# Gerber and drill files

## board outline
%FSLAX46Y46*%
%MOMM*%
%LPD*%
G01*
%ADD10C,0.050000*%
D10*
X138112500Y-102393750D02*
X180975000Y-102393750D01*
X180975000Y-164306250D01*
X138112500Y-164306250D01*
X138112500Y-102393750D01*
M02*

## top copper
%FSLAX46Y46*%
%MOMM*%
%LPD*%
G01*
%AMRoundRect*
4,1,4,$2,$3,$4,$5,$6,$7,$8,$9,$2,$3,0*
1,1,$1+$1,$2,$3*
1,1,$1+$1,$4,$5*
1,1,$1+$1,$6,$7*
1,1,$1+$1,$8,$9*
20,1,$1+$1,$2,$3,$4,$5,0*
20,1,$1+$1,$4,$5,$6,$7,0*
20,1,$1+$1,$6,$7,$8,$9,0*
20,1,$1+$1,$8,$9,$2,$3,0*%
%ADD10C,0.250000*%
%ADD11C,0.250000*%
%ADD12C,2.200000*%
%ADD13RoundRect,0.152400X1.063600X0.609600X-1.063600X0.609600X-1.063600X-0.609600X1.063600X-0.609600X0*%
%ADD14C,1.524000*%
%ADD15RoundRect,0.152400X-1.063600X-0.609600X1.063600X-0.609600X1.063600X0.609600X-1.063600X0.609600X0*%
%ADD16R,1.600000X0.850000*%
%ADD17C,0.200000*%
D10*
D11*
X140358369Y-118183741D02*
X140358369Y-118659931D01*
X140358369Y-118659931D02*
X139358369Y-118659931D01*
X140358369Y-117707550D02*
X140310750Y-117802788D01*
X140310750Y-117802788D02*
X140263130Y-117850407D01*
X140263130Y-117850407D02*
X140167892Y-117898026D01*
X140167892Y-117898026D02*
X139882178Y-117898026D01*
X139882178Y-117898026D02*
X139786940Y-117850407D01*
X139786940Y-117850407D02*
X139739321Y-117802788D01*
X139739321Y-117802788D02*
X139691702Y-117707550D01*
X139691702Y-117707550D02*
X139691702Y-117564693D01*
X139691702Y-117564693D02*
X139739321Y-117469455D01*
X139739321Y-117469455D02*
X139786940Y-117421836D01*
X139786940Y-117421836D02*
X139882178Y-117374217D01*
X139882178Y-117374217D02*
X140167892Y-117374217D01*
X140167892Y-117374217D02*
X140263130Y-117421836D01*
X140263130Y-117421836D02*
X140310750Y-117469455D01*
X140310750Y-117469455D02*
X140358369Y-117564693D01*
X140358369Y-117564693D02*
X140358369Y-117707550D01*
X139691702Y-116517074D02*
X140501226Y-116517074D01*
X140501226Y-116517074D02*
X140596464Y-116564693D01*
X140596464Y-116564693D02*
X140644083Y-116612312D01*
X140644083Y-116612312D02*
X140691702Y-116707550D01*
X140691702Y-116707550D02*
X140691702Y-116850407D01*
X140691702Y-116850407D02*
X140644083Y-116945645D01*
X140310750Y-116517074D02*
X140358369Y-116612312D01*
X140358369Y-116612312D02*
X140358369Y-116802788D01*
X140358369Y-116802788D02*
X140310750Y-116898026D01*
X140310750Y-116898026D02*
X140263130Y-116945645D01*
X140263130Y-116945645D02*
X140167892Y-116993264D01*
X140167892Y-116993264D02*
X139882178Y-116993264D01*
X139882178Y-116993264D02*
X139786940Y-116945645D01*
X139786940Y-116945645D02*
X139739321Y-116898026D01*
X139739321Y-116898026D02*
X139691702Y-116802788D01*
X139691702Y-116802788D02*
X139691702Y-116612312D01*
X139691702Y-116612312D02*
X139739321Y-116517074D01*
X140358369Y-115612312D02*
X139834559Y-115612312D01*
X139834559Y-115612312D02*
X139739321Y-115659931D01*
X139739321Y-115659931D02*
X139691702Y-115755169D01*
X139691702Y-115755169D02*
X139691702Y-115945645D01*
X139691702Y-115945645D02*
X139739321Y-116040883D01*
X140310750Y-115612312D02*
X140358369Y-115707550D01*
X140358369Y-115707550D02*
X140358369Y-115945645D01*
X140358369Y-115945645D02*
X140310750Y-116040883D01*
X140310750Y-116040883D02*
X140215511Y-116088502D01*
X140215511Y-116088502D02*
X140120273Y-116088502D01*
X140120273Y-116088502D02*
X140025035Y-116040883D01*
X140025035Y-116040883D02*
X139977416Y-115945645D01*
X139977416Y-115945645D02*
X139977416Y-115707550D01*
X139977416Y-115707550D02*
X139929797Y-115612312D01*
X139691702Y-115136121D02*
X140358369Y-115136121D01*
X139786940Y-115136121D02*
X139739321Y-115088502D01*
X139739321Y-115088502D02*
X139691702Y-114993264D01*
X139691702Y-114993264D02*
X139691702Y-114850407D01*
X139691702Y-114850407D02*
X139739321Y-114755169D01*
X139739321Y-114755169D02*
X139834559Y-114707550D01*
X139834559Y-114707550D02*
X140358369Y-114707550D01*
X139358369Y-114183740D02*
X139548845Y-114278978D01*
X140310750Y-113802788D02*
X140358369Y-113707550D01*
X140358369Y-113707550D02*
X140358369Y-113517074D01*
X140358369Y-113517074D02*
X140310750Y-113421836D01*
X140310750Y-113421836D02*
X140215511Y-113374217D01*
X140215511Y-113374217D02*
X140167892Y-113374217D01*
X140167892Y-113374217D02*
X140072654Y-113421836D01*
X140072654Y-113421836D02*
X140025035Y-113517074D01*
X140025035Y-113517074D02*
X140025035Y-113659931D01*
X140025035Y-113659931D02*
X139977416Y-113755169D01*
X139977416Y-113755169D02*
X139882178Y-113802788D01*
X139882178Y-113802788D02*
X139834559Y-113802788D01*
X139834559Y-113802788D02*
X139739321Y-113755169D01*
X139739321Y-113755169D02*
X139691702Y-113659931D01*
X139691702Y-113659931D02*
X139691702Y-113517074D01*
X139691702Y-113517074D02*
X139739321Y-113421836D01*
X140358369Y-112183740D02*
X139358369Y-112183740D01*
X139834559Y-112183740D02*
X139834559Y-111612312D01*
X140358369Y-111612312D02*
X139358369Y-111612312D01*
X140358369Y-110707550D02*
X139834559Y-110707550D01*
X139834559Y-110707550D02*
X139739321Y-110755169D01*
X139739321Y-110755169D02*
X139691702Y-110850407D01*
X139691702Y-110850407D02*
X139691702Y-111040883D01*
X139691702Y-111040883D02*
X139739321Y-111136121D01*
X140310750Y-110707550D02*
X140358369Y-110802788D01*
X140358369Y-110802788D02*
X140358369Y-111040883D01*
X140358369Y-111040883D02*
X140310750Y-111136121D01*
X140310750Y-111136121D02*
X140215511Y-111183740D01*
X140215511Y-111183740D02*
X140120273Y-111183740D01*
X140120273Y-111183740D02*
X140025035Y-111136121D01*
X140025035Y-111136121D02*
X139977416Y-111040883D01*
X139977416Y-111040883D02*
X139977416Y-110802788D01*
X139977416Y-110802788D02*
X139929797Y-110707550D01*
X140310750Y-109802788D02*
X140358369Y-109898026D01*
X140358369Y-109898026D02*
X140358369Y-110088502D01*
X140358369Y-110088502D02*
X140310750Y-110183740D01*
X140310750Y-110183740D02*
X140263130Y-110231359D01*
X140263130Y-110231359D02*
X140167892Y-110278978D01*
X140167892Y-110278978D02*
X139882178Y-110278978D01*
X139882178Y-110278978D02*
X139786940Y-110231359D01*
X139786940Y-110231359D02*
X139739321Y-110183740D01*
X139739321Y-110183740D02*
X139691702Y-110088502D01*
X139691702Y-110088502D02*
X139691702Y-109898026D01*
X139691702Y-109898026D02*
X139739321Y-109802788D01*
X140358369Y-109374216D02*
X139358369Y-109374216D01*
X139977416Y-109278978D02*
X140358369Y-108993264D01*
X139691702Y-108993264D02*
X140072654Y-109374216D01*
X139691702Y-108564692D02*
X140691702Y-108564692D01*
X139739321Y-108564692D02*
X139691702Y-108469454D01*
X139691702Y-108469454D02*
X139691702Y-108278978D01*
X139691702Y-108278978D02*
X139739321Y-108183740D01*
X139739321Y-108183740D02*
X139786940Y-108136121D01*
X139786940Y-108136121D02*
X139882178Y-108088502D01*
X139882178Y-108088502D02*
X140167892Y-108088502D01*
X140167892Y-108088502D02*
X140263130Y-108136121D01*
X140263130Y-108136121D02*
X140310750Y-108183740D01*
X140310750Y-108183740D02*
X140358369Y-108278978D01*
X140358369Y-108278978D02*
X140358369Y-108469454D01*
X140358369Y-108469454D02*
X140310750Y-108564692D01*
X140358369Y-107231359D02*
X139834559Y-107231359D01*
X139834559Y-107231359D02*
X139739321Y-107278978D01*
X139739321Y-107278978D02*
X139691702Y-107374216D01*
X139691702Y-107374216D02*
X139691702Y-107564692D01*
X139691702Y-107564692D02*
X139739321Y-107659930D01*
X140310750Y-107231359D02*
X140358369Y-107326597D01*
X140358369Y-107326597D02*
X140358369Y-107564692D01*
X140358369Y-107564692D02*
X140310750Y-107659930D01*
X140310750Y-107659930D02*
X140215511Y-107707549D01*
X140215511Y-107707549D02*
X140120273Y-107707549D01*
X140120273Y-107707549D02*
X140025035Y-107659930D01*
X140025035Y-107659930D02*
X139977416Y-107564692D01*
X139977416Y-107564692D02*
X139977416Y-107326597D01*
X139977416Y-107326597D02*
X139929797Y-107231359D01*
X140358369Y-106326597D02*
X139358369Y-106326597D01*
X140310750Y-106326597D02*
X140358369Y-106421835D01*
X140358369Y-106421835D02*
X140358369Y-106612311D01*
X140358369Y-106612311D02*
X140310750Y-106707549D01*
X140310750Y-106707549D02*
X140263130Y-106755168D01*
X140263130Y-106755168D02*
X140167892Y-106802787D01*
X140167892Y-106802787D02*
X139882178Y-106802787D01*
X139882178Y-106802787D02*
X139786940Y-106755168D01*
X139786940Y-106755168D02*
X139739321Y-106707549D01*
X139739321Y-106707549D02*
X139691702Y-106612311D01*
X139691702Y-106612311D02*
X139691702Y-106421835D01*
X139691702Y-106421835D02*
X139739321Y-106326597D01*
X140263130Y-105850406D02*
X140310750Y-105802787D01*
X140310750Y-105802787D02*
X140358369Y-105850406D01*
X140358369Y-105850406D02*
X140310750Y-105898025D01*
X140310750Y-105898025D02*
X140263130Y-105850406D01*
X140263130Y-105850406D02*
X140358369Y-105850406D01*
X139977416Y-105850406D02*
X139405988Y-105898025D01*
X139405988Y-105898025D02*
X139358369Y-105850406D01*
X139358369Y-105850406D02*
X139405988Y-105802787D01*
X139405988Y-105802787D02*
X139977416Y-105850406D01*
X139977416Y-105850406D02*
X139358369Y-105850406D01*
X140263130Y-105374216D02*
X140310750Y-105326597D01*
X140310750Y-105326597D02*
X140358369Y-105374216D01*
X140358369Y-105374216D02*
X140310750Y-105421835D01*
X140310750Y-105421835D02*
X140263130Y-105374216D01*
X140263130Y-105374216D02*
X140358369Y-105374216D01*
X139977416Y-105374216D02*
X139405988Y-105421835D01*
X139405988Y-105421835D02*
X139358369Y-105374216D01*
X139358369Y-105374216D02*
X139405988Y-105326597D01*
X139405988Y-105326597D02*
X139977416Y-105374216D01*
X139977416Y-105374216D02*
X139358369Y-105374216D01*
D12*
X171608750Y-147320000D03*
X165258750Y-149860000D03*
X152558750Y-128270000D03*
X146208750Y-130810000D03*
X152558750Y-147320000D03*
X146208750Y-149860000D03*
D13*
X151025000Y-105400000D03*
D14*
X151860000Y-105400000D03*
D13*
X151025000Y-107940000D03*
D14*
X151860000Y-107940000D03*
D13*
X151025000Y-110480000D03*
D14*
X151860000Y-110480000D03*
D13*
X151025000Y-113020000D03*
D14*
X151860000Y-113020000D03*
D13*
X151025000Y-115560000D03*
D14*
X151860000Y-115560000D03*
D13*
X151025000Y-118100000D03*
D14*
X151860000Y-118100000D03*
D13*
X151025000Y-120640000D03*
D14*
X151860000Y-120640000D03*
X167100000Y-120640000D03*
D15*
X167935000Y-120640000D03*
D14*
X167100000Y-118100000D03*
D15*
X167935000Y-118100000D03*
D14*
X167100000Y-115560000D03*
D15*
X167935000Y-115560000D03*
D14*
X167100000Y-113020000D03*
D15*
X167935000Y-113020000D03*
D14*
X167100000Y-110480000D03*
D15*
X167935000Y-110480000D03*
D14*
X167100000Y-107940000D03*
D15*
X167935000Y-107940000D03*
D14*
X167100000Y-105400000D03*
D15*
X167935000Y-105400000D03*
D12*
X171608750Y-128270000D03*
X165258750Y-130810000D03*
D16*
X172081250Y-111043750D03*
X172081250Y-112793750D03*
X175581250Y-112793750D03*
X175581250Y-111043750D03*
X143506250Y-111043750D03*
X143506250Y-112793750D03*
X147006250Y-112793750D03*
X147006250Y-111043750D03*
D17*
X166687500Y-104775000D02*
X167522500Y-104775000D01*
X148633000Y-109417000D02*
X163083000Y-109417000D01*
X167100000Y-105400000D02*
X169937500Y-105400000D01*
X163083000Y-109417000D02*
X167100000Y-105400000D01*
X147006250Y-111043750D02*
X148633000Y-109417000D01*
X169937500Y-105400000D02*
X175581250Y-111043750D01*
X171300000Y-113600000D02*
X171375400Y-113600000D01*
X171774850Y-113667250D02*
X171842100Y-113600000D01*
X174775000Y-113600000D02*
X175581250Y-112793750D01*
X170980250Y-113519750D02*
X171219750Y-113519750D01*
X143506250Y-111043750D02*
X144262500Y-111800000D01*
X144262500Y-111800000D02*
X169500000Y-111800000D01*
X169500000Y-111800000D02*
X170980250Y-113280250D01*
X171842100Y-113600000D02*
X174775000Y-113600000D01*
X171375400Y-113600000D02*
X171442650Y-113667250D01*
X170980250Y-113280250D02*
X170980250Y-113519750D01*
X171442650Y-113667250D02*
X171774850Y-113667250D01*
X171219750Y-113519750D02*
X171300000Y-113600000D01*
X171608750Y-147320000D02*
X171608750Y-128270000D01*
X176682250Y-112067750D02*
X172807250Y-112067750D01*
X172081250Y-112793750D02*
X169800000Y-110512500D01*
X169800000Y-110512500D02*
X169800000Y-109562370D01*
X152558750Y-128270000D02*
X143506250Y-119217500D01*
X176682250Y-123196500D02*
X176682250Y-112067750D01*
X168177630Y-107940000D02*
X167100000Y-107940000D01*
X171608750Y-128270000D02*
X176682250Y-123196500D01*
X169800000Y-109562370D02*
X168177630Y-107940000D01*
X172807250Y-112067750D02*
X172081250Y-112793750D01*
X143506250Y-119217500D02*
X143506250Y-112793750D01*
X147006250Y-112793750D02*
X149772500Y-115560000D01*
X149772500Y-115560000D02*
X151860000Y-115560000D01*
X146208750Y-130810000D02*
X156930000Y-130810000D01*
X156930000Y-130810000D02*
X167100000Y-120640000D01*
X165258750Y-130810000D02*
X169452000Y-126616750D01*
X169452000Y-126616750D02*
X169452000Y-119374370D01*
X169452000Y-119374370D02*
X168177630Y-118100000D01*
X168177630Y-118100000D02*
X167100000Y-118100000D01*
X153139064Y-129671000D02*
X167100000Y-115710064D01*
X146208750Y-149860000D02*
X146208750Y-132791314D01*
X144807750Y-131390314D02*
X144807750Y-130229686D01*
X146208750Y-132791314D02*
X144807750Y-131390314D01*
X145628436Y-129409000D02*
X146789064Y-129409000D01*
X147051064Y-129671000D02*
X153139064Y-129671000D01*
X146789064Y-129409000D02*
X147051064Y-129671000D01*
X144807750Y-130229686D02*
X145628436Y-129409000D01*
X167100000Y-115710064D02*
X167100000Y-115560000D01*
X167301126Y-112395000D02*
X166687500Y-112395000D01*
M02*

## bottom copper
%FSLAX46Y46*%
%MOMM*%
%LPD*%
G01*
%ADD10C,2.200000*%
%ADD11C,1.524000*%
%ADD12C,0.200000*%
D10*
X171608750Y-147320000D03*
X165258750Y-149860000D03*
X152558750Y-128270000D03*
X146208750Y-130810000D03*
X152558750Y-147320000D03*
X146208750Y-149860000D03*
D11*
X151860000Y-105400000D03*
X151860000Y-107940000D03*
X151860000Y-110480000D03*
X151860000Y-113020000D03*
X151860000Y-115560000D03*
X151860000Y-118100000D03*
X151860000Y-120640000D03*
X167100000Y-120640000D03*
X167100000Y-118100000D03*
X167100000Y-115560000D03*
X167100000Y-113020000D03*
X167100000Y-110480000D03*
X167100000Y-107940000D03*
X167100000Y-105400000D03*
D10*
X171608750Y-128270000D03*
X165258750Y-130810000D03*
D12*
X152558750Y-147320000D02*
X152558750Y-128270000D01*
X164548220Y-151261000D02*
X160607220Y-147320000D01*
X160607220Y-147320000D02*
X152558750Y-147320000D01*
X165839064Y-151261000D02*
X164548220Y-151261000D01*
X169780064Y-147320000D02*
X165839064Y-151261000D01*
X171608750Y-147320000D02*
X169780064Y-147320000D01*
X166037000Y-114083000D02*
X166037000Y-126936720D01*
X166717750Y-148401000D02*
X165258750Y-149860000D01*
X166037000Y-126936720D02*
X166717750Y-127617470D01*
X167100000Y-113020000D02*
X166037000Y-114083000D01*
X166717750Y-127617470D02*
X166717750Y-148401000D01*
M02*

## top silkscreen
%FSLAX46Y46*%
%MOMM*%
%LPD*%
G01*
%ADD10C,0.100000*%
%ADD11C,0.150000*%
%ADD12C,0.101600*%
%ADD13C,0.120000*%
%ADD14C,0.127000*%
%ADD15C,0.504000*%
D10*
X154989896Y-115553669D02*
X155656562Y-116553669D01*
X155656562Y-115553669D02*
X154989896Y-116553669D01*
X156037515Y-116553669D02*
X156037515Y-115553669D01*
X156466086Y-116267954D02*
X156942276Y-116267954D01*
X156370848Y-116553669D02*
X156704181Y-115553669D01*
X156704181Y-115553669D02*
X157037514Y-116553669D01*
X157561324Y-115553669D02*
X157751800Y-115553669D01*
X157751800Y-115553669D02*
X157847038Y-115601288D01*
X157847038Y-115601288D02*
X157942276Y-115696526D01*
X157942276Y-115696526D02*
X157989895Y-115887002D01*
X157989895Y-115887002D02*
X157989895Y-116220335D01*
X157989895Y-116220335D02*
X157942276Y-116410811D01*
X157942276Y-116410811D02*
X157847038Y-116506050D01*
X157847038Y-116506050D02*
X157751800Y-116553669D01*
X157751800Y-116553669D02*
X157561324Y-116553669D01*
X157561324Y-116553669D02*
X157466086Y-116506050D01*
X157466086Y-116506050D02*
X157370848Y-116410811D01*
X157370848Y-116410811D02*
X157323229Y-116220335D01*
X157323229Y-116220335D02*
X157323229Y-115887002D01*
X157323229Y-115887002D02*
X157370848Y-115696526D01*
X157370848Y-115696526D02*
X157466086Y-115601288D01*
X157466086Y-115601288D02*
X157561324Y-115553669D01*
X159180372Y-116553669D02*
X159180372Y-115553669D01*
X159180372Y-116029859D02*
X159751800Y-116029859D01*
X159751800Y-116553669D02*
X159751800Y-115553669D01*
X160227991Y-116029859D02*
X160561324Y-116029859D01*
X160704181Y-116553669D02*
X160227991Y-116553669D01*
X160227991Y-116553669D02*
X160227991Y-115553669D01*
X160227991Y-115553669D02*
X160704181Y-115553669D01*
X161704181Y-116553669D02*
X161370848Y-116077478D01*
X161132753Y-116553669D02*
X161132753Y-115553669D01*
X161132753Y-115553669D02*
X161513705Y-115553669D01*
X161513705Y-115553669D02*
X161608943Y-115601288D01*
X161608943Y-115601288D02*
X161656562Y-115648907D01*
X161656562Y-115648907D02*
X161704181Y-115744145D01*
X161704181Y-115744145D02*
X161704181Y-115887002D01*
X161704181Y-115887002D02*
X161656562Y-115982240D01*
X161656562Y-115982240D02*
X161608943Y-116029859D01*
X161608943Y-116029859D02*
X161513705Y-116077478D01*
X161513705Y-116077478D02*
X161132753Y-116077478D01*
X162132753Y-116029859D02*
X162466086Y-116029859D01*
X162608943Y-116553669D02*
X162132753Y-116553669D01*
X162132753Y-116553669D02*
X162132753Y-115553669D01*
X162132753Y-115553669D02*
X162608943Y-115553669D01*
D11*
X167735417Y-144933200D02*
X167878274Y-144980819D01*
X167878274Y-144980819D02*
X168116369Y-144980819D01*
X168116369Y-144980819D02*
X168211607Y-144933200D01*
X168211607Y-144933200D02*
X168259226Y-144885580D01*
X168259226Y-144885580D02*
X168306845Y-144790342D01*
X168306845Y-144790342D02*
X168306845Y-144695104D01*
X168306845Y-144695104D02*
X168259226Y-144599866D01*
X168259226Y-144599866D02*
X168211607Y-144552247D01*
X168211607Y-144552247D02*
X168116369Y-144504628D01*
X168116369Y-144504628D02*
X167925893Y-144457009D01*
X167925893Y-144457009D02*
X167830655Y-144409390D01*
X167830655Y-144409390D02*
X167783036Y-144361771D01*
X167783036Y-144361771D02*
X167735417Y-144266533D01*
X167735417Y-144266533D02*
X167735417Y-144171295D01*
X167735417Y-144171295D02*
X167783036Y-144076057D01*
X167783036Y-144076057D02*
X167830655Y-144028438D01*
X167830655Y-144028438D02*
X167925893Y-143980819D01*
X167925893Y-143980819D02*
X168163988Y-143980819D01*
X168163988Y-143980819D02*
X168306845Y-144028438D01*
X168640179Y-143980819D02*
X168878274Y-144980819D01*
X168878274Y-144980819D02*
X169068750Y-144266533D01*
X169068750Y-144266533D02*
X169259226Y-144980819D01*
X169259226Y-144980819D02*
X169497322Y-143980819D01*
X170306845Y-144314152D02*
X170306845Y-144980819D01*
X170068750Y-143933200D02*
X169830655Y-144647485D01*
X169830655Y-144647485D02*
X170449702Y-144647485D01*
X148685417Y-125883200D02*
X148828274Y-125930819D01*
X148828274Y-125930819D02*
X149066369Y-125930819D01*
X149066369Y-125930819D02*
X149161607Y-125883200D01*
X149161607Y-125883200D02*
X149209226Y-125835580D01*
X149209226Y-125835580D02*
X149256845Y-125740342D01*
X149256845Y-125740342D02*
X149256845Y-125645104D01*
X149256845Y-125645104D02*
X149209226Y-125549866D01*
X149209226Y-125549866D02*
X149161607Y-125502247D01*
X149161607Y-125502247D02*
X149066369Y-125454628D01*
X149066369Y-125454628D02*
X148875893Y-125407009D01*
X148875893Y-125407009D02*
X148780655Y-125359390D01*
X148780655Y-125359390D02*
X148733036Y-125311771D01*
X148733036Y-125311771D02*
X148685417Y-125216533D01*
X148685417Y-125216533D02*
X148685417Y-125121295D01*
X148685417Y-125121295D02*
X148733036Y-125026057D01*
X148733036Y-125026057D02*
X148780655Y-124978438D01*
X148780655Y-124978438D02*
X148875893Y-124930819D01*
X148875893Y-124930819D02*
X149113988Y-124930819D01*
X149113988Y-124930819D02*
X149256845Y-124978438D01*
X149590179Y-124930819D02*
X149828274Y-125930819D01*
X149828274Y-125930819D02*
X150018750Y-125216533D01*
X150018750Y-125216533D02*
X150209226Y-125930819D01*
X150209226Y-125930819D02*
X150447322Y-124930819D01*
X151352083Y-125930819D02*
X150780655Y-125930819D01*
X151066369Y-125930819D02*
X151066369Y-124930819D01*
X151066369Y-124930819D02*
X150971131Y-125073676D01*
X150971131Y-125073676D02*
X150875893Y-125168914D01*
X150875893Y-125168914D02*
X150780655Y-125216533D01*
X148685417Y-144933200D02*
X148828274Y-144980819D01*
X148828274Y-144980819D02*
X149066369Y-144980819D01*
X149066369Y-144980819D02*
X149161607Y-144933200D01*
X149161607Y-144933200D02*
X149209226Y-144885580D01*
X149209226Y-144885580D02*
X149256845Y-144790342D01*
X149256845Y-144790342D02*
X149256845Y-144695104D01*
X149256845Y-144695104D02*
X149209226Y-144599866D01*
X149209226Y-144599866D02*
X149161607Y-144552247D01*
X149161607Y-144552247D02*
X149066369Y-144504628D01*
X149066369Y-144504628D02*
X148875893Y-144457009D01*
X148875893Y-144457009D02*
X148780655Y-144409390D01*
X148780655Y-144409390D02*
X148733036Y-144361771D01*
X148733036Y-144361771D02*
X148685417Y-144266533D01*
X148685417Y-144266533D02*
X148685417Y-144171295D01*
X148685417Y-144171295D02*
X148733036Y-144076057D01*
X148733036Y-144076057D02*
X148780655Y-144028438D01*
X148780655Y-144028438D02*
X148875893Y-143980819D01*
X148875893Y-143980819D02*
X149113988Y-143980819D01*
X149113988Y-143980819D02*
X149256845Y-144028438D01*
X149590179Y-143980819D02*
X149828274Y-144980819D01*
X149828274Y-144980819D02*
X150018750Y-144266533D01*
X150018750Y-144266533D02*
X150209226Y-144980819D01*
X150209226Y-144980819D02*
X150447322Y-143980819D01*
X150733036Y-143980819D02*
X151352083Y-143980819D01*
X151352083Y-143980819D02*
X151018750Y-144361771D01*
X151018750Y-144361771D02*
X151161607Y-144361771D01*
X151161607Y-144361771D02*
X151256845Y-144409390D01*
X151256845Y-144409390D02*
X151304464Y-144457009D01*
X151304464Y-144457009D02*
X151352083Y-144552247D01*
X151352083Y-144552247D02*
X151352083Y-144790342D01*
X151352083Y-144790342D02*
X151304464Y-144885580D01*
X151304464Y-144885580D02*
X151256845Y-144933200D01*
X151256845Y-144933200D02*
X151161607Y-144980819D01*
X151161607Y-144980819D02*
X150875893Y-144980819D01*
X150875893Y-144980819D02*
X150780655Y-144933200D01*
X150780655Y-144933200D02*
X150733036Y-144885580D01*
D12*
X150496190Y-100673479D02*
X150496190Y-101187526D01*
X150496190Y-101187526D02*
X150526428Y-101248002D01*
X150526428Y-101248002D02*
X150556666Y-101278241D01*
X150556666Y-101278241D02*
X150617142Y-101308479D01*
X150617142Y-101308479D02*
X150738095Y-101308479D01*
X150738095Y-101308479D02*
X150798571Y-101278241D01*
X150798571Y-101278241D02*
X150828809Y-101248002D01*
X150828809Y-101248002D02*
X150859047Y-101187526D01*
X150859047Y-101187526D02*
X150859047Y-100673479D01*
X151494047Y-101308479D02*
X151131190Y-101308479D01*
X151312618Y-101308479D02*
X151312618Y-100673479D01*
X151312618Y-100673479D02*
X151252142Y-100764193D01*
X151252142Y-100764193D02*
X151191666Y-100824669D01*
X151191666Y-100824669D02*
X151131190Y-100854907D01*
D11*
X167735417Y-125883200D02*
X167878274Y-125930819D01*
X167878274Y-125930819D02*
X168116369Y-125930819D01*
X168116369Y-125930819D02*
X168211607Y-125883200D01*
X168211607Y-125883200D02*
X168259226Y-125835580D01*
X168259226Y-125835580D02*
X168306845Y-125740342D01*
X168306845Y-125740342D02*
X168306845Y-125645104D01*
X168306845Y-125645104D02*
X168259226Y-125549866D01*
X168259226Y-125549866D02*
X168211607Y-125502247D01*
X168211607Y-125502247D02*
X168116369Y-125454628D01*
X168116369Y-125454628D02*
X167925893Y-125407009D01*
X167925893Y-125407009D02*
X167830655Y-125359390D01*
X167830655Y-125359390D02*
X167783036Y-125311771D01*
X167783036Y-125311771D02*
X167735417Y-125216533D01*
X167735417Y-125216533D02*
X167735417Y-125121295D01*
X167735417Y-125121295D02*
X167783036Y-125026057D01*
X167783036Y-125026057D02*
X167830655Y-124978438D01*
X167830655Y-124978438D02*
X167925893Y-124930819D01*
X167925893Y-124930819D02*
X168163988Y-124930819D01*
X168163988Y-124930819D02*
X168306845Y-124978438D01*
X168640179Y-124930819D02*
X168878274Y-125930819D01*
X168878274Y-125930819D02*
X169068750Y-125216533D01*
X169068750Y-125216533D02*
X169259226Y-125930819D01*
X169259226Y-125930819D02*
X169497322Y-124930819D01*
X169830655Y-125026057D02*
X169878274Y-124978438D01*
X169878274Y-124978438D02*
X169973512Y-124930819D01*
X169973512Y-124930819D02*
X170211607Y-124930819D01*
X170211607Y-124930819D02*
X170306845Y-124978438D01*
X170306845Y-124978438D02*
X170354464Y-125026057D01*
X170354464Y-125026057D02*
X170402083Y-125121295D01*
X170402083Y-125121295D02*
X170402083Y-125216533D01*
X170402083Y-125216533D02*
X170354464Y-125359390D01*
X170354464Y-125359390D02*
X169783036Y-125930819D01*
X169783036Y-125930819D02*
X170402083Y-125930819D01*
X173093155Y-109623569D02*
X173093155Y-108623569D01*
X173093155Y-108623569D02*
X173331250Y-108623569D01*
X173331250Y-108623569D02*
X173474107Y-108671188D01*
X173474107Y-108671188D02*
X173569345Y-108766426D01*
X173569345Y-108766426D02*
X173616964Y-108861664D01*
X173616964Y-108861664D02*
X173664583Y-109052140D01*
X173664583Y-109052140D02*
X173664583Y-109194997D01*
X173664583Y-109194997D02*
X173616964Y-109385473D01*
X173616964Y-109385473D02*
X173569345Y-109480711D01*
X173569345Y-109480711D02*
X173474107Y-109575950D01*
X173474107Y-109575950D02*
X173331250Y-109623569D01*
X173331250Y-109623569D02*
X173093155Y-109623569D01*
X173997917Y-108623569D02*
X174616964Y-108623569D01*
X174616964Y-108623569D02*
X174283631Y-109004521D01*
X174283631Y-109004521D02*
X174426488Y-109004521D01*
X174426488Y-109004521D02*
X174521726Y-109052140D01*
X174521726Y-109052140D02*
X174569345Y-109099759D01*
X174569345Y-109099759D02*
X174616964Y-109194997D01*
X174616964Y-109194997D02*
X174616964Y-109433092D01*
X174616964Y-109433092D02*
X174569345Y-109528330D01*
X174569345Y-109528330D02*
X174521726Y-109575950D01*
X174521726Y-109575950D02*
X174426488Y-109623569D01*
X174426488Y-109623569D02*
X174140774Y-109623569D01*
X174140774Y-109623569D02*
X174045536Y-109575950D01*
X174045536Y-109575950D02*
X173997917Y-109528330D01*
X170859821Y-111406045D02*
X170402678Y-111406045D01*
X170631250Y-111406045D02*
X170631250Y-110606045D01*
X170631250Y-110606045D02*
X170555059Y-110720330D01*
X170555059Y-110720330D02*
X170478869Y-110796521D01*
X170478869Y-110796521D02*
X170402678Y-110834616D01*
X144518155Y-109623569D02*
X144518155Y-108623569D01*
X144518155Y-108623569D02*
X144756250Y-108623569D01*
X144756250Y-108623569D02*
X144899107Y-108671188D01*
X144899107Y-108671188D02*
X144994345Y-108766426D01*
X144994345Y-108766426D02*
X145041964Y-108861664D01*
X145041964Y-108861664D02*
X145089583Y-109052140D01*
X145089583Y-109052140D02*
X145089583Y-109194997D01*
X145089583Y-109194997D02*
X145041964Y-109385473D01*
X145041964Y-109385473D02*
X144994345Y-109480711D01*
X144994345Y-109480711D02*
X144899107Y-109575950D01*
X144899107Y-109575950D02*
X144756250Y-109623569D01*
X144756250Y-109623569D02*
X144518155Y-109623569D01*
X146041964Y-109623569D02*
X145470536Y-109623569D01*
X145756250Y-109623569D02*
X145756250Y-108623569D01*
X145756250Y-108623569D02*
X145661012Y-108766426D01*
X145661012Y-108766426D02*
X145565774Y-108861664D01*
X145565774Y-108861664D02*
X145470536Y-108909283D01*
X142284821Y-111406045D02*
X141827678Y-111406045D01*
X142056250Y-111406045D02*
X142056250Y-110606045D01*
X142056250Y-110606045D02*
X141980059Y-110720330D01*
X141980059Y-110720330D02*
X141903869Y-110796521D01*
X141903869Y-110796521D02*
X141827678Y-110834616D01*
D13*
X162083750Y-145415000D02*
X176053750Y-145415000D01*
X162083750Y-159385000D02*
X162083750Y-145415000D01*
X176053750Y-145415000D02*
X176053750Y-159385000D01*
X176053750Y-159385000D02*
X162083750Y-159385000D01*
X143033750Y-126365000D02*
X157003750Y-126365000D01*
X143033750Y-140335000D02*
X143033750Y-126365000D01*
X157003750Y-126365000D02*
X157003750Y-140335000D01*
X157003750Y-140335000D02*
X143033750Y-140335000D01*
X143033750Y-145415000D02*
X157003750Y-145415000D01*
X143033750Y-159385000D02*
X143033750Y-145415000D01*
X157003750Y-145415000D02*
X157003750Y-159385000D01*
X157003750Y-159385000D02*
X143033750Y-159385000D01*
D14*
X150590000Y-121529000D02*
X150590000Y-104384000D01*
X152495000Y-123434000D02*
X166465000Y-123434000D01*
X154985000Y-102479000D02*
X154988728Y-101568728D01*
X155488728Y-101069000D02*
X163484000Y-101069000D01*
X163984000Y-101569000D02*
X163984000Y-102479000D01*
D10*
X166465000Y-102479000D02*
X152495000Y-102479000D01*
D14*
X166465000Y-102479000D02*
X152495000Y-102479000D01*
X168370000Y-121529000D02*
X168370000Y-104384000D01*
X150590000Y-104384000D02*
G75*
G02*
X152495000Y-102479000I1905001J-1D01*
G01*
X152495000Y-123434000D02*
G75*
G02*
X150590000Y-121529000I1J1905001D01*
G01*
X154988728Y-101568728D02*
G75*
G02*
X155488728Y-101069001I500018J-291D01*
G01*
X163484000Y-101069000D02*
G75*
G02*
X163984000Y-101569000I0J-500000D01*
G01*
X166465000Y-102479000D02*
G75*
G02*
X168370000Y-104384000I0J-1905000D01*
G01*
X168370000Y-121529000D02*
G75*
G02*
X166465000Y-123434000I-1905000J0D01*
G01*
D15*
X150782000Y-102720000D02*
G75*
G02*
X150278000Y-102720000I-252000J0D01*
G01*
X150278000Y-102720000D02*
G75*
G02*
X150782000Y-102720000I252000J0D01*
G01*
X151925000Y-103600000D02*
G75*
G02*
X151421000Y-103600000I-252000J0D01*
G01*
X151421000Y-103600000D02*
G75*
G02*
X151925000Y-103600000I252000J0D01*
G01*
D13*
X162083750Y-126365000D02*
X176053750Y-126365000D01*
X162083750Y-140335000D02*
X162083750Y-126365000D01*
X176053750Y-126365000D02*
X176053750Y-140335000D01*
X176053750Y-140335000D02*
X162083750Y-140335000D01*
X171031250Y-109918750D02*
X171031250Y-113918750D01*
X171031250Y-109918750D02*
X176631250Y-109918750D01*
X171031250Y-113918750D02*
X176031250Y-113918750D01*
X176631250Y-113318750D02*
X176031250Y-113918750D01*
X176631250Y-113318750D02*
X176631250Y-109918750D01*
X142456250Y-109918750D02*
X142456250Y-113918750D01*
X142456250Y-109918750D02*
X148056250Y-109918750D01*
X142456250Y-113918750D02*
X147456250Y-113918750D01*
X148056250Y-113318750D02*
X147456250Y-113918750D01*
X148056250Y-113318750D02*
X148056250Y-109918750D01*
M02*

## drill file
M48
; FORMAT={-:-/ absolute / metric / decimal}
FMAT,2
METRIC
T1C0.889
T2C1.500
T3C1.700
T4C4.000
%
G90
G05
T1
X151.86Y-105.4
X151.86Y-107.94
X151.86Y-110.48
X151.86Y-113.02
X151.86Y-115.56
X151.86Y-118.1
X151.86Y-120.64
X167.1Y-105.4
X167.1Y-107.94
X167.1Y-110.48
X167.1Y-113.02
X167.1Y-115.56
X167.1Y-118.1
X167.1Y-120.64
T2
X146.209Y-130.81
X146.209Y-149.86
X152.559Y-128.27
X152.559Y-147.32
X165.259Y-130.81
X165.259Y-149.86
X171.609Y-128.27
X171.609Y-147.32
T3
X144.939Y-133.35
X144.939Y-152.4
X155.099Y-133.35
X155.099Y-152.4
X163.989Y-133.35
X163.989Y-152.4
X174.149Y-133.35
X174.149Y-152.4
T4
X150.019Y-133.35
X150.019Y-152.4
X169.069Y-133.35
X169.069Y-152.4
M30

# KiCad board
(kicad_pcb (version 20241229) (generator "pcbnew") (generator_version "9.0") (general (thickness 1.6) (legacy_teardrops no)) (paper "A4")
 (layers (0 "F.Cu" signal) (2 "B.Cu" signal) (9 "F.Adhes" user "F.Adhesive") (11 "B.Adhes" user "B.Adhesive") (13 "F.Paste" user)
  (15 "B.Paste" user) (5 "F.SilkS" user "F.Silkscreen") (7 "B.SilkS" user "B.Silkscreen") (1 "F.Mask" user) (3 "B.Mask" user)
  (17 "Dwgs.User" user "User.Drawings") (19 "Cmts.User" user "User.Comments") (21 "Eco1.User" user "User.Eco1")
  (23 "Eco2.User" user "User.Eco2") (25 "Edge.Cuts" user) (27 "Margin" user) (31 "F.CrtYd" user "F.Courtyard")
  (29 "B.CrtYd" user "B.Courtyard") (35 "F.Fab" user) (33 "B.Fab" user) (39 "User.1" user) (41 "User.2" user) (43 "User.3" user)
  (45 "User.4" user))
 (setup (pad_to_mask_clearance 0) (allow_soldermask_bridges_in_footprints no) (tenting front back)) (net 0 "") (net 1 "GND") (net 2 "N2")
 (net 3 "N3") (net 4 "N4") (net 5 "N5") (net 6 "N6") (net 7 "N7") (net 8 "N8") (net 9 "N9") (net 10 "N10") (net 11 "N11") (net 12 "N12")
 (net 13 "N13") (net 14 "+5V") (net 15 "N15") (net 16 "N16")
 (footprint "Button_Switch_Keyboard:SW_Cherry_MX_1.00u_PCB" (layer "F.Cu") (at 171.60875 147.32)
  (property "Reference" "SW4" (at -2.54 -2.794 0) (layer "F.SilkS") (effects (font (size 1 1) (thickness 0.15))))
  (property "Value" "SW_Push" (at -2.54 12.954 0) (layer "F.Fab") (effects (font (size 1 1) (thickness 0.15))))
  (fp_line (start -9.525 -1.905) (end 4.445 -1.905) (stroke (width 0.12) (type solid)) (layer "F.SilkS"))
  (fp_line (start -9.525 12.065) (end -9.525 -1.905) (stroke (width 0.12) (type solid)) (layer "F.SilkS"))
  (fp_line (start 4.445 -1.905) (end 4.445 12.065) (stroke (width 0.12) (type solid)) (layer "F.SilkS"))
  (fp_line (start 4.445 12.065) (end -9.525 12.065) (stroke (width 0.12) (type solid)) (layer "F.SilkS"))
  (pad "" np_thru_hole circle (at -7.62 5.08) (size 1.7 1.7) (drill 1.7) (layers "*.Cu" "*.Mask"))
  (pad "" np_thru_hole circle (at -2.54 5.08) (size 4 4) (drill 4) (layers "*.Cu" "*.Mask"))
  (pad "" np_thru_hole circle (at 2.54 5.08) (size 1.7 1.7) (drill 1.7) (layers "*.Cu" "*.Mask"))
  (pad "1" thru_hole circle (at 0 0) (size 2.2 2.2) (drill 1.5) (layers "*.Cu" "*.Mask") (remove_unused_layers no) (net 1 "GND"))
  (pad "2" thru_hole circle (at -6.35 2.54) (size 2.2 2.2) (drill 1.5) (layers "*.Cu" "*.Mask") (remove_unused_layers no) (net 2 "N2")))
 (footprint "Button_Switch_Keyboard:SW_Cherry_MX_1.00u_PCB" (layer "F.Cu") (at 152.55875 128.27)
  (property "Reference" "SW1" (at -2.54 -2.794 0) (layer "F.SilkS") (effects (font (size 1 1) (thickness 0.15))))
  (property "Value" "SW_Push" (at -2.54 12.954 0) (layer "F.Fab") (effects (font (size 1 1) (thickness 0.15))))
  (fp_line (start -9.525 -1.905) (end 4.445 -1.905) (stroke (width 0.12) (type solid)) (layer "F.SilkS"))
  (fp_line (start -9.525 12.065) (end -9.525 -1.905) (stroke (width 0.12) (type solid)) (layer "F.SilkS"))
  (fp_line (start 4.445 -1.905) (end 4.445 12.065) (stroke (width 0.12) (type solid)) (layer "F.SilkS"))
  (fp_line (start 4.445 12.065) (end -9.525 12.065) (stroke (width 0.12) (type solid)) (layer "F.SilkS"))
  (pad "" np_thru_hole circle (at -7.62 5.08) (size 1.7 1.7) (drill 1.7) (layers "*.Cu" "*.Mask"))
  (pad "" np_thru_hole circle (at -2.54 5.08) (size 4 4) (drill 4) (layers "*.Cu" "*.Mask"))
  (pad "" np_thru_hole circle (at 2.54 5.08) (size 1.7 1.7) (drill 1.7) (layers "*.Cu" "*.Mask"))
  (pad "1" thru_hole circle (at 0 0) (size 2.2 2.2) (drill 1.5) (layers "*.Cu" "*.Mask") (remove_unused_layers no) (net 1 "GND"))
  (pad "2" thru_hole circle (at -6.35 2.54) (size 2.2 2.2) (drill 1.5) (layers "*.Cu" "*.Mask") (remove_unused_layers no) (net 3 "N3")))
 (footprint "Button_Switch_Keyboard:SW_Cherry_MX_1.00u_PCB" (layer "F.Cu") (at 152.55875 147.32)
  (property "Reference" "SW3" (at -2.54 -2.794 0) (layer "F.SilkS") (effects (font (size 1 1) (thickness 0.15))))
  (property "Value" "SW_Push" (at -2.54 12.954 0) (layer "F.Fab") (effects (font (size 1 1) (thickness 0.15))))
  (fp_line (start -9.525 -1.905) (end 4.445 -1.905) (stroke (width 0.12) (type solid)) (layer "F.SilkS"))
  (fp_line (start -9.525 12.065) (end -9.525 -1.905) (stroke (width 0.12) (type solid)) (layer "F.SilkS"))
  (fp_line (start 4.445 -1.905) (end 4.445 12.065) (stroke (width 0.12) (type solid)) (layer "F.SilkS"))
  (fp_line (start 4.445 12.065) (end -9.525 12.065) (stroke (width 0.12) (type solid)) (layer "F.SilkS"))
  (pad "" np_thru_hole circle (at -7.62 5.08) (size 1.7 1.7) (drill 1.7) (layers "*.Cu" "*.Mask"))
  (pad "" np_thru_hole circle (at -2.54 5.08) (size 4 4) (drill 4) (layers "*.Cu" "*.Mask"))
  (pad "" np_thru_hole circle (at 2.54 5.08) (size 1.7 1.7) (drill 1.7) (layers "*.Cu" "*.Mask"))
  (pad "1" thru_hole circle (at 0 0) (size 2.2 2.2) (drill 1.5) (layers "*.Cu" "*.Mask") (remove_unused_layers no) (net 1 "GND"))
  (pad "2" thru_hole circle (at -6.35 2.54) (size 2.2 2.2) (drill 1.5) (layers "*.Cu" "*.Mask") (remove_unused_layers no) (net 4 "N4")))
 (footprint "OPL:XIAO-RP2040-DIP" (layer "F.Cu") (at 159.48 113.02)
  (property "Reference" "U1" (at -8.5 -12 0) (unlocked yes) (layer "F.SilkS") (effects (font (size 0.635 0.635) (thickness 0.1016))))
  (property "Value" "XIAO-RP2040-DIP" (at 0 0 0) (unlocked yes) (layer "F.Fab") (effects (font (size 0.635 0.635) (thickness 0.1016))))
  (fp_line (start -8.89 8.509) (end -8.89 -8.636) (stroke (width 0.127) (type solid)) (layer "F.SilkS"))
  (fp_line (start -6.985 10.414) (end 6.985 10.414) (stroke (width 0.127) (type solid)) (layer "F.SilkS"))
  (fp_line (start -4.495 -10.541) (end -4.491272 -11.451272) (stroke (width 0.127) (type solid)) (layer "F.SilkS"))
  (fp_line (start -3.991272 -11.951) (end 4.004 -11.951) (stroke (width 0.127) (type solid)) (layer "F.SilkS"))
  (fp_line (start 4.504 -11.451) (end 4.504 -10.541) (stroke (width 0.127) (type solid)) (layer "F.SilkS"))
  (fp_line (start 6.985 -10.541) (end -6.985 -10.541) (stroke (width 0.1) (type solid)) (layer "F.SilkS"))
  (fp_line (start 6.985 -10.541) (end -6.985 -10.541) (stroke (width 0.127) (type solid)) (layer "F.SilkS"))
  (fp_line (start 8.89 8.509) (end 8.89 -8.636) (stroke (width 0.127) (type solid)) (layer "F.SilkS"))
  (fp_arc (start -8.89 -8.636) (mid -8.332038 -9.983038) (end -6.985 -10.541) (stroke (width 0.127) (type solid)) (layer "F.SilkS"))
  (fp_arc (start -6.985 10.414) (mid -8.332038 9.856038) (end -8.89 8.509) (stroke (width 0.127) (type solid)) (layer "F.SilkS"))
  (fp_arc (start -4.491272 -11.451272) (mid -4.344728 -11.80464) (end -3.991272 -11.951) (stroke (width 0.127) (type default))
   (layer "F.SilkS"))
  (fp_arc (start 4.004 -11.951) (mid 4.357553 -11.804553) (end 4.504 -11.451) (stroke (width 0.127) (type default)) (layer "F.SilkS"))
  (fp_arc (start 6.985 -10.541) (mid 8.332038 -9.983038) (end 8.89 -8.636) (stroke (width 0.127) (type solid)) (layer "F.SilkS"))
  (fp_arc (start 8.89 8.509) (mid 8.332038 9.856038) (end 6.985 10.414) (stroke (width 0.127) (type solid)) (layer "F.SilkS"))
  (fp_circle (center -8.95 -10.3) (end -8.95 -10.554) (stroke (width 0.5) (type solid)) (fill yes) (layer "F.SilkS"))
  (fp_circle (center -7.807 -9.42) (end -7.807 -9.674) (stroke (width 0.5) (type solid)) (fill yes) (layer "F.SilkS"))
  (pad "1" smd roundrect (at -8.455 -7.62 180) (size 2.432 1.524) (layers "F.Cu" "F.Mask") (roundrect_rratio 0.1) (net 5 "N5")
   (thermal_bridge_angle 45))
  (pad "1" thru_hole circle (at -7.62 -7.62 180) (size 1.524 1.524) (drill 0.889) (layers "*.Cu" "*.Mask") (remove_unused_layers no)
   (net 5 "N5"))
  (pad "2" smd roundrect (at -8.455 -5.08 180) (size 2.432 1.524) (layers "F.Cu" "F.Mask") (roundrect_rratio 0.1) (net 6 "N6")
   (thermal_bridge_angle 45))
  (pad "2" thru_hole circle (at -7.62 -5.08 180) (size 1.524 1.524) (drill 0.889) (layers "*.Cu" "*.Mask") (remove_unused_layers no)
   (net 6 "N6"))
  (pad "3" smd roundrect (at -8.455 -2.54 180) (size 2.432 1.524) (layers "F.Cu" "F.Mask") (roundrect_rratio 0.1) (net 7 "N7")
   (thermal_bridge_angle 45))
  (pad "3" thru_hole circle (at -7.62 -2.54 180) (size 1.524 1.524) (drill 0.889) (layers "*.Cu" "*.Mask") (remove_unused_layers no)
   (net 7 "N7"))
  (pad "4" smd roundrect (at -8.455 0 180) (size 2.432 1.524) (layers "F.Cu" "F.Mask") (roundrect_rratio 0.1) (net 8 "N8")
   (thermal_bridge_angle 45))
  (pad "4" thru_hole circle (at -7.62 0 180) (size 1.524 1.524) (drill 0.889) (layers "*.Cu" "*.Mask") (remove_unused_layers no)
   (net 8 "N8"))
  (pad "5" smd roundrect (at -8.455 2.54 180) (size 2.432 1.524) (layers "F.Cu" "F.Mask") (roundrect_rratio 0.1) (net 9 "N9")
   (thermal_bridge_angle 45))
  (pad "5" thru_hole circle (at -7.62 2.54 180) (size 1.524 1.524) (drill 0.889) (layers "*.Cu" "*.Mask") (remove_unused_layers no)
   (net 9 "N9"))
  (pad "6" smd roundrect (at -8.455 5.08 180) (size 2.432 1.524) (layers "F.Cu" "F.Mask") (roundrect_rratio 0.1) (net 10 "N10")
   (thermal_bridge_angle 45))
  (pad "6" thru_hole circle (at -7.62 5.08 180) (size 1.524 1.524) (drill 0.889) (layers "*.Cu" "*.Mask") (remove_unused_layers no)
   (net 10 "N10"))
  (pad "7" smd roundrect (at -8.455 7.62 180) (size 2.432 1.524) (layers "F.Cu" "F.Mask") (roundrect_rratio 0.1) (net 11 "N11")
   (thermal_bridge_angle 45))
  (pad "7" thru_hole circle (at -7.62 7.62 180) (size 1.524 1.524) (drill 0.889) (layers "*.Cu" "*.Mask") (remove_unused_layers no)
   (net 11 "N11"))
  (pad "8" thru_hole circle (at 7.62 7.62) (size 1.524 1.524) (drill 0.889) (layers "*.Cu" "*.Mask") (remove_unused_layers no) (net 3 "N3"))
  (pad "8" smd roundrect (at 8.455 7.62) (size 2.432 1.524) (layers "F.Cu" "F.Mask") (roundrect_rratio 0.1) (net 3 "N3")
   (thermal_bridge_angle 45))
  (pad "9" thru_hole circle (at 7.62 5.08) (size 1.524 1.524) (drill 0.889) (layers "*.Cu" "*.Mask") (remove_unused_layers no)
   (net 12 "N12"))
  (pad "9" smd roundrect (at 8.455 5.08) (size 2.432 1.524) (layers "F.Cu" "F.Mask") (roundrect_rratio 0.1) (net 12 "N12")
   (thermal_bridge_angle 45))
  (pad "10" thru_hole circle (at 7.62 2.54) (size 1.524 1.524) (drill 0.889) (layers "*.Cu" "*.Mask") (remove_unused_layers no) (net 4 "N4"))
  (pad "10" smd roundrect (at 8.455 2.54) (size 2.432 1.524) (layers "F.Cu" "F.Mask") (roundrect_rratio 0.1) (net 4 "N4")
   (thermal_bridge_angle 45))
  (pad "11" thru_hole circle (at 7.62 0) (size 1.524 1.524) (drill 0.889) (layers "*.Cu" "*.Mask") (remove_unused_layers no) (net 2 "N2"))
  (pad "11" smd roundrect (at 8.455 0) (size 2.432 1.524) (layers "F.Cu" "F.Mask") (roundrect_rratio 0.1) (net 2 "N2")
   (thermal_bridge_angle 45))
  (pad "12" thru_hole circle (at 7.62 -2.54) (size 1.524 1.524) (drill 0.889) (layers "*.Cu" "*.Mask") (remove_unused_layers no)
   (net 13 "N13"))
  (pad "12" smd roundrect (at 8.455 -2.54) (size 2.432 1.524) (layers "F.Cu" "F.Mask") (roundrect_rratio 0.1) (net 13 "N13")
   (thermal_bridge_angle 45))
  (pad "13" thru_hole circle (at 7.62 -5.08) (size 1.524 1.524) (drill 0.889) (layers "*.Cu" "*.Mask") (remove_unused_layers no)
   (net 1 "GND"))
  (pad "13" smd roundrect (at 8.455 -5.08) (size 2.432 1.524) (layers "F.Cu" "F.Mask") (roundrect_rratio 0.1) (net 1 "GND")
   (thermal_bridge_angle 45))
  (pad "14" thru_hole circle (at 7.62 -7.62) (size 1.524 1.524) (drill 0.889) (layers "*.Cu" "*.Mask") (remove_unused_layers no)
   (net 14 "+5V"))
  (pad "14" smd roundrect (at 8.455 -7.62) (size 2.432 1.524) (layers "F.Cu" "F.Mask") (roundrect_rratio 0.1) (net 14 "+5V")
   (thermal_bridge_angle 45)))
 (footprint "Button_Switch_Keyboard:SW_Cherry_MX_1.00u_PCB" (layer "F.Cu") (at 171.60875 128.27)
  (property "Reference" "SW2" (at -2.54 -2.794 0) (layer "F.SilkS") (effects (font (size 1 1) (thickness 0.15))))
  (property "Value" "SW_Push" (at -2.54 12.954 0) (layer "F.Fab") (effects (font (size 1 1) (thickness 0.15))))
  (fp_line (start -9.525 -1.905) (end 4.445 -1.905) (stroke (width 0.12) (type solid)) (layer "F.SilkS"))
  (fp_line (start -9.525 12.065) (end -9.525 -1.905) (stroke (width 0.12) (type solid)) (layer "F.SilkS"))
  (fp_line (start 4.445 -1.905) (end 4.445 12.065) (stroke (width 0.12) (type solid)) (layer "F.SilkS"))
  (fp_line (start 4.445 12.065) (end -9.525 12.065) (stroke (width 0.12) (type solid)) (layer "F.SilkS"))
  (pad "" np_thru_hole circle (at -7.62 5.08) (size 1.7 1.7) (drill 1.7) (layers "*.Cu" "*.Mask"))
  (pad "" np_thru_hole circle (at -2.54 5.08) (size 4 4) (drill 4) (layers "*.Cu" "*.Mask"))
  (pad "" np_thru_hole circle (at 2.54 5.08) (size 1.7 1.7) (drill 1.7) (layers "*.Cu" "*.Mask"))
  (pad "1" thru_hole circle (at 0 0) (size 2.2 2.2) (drill 1.5) (layers "*.Cu" "*.Mask") (remove_unused_layers no) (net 1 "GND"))
  (pad "2" thru_hole circle (at -6.35 2.54) (size 2.2 2.2) (drill 1.5) (layers "*.Cu" "*.Mask") (remove_unused_layers no) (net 12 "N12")))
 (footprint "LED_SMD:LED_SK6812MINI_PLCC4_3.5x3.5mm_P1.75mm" (layer "F.Cu") (at 173.83125 111.91875)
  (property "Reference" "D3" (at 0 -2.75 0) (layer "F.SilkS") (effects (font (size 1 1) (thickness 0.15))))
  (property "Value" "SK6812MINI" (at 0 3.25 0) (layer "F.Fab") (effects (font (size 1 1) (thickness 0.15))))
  (fp_line (start -2.8 -2) (end -2.8 2) (stroke (width 0.12) (type default)) (layer "F.SilkS"))
  (fp_line (start -2.8 -2) (end 2.8 -2) (stroke (width 0.12) (type solid)) (layer "F.SilkS"))
  (fp_line (start -2.8 2) (end 2.2 2) (stroke (width 0.12) (type solid)) (layer "F.SilkS"))
  (fp_line (start 2.8 1.4) (end 2.2 2) (stroke (width 0.12) (type default)) (layer "F.SilkS"))
  (fp_line (start 2.8 1.4) (end 2.8 -2) (stroke (width 0.12) (type solid)) (layer "F.SilkS"))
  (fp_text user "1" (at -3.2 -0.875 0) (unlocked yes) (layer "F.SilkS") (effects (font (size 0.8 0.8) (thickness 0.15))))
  (pad "1" smd rect (at -1.75 -0.875) (size 1.6 0.85) (layers "F.Cu" "F.Mask" "F.Paste") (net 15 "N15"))
  (pad "2" smd rect (at -1.75 0.875) (size 1.6 0.85) (layers "F.Cu" "F.Mask" "F.Paste") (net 1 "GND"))
  (pad "3" smd rect (at 1.75 0.875) (size 1.6 0.85) (layers "F.Cu" "F.Mask" "F.Paste") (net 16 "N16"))
  (pad "4" smd rect (at 1.75 -0.875) (size 1.6 0.85) (layers "F.Cu" "F.Mask" "F.Paste") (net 14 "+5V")))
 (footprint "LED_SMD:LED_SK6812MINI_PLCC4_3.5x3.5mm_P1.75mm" (layer "F.Cu") (at 145.25625 111.91875)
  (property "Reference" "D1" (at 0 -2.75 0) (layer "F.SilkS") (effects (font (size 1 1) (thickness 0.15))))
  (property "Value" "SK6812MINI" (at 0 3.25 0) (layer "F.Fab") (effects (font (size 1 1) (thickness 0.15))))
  (fp_line (start -2.8 -2) (end -2.8 2) (stroke (width 0.12) (type default)) (layer "F.SilkS"))
  (fp_line (start -2.8 -2) (end 2.8 -2) (stroke (width 0.12) (type solid)) (layer "F.SilkS"))
  (fp_line (start -2.8 2) (end 2.2 2) (stroke (width 0.12) (type solid)) (layer "F.SilkS"))
  (fp_line (start 2.8 1.4) (end 2.2 2) (stroke (width 0.12) (type default)) (layer "F.SilkS"))
  (fp_line (start 2.8 1.4) (end 2.8 -2) (stroke (width 0.12) (type solid)) (layer "F.SilkS"))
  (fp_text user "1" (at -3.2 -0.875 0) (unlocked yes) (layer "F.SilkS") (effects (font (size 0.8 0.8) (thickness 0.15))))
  (pad "1" smd rect (at -1.75 -0.875) (size 1.6 0.85) (layers "F.Cu" "F.Mask" "F.Paste") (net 16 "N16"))
  (pad "2" smd rect (at -1.75 0.875) (size 1.6 0.85) (layers "F.Cu" "F.Mask" "F.Paste") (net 1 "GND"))
  (pad "3" smd rect (at 1.75 0.875) (size 1.6 0.85) (layers "F.Cu" "F.Mask" "F.Paste") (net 9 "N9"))
  (pad "4" smd rect (at 1.75 -0.875) (size 1.6 0.85) (layers "F.Cu" "F.Mask" "F.Paste") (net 14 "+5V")))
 (gr_rect (start 138.1125 102.39375) (end 180.975 164.30625) (stroke (width 0.05) (type default)) (fill no) (layer "Edge.Cuts"))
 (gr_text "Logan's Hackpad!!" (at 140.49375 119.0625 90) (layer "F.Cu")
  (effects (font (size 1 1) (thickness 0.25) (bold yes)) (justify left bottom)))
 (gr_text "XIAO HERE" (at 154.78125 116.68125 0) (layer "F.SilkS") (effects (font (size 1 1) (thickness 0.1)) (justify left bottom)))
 (segment (start 166.6875 104.775) (end 167.5225 104.775) (width 0.2) (layer "F.Cu") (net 14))
 (segment (start 148.633 109.417) (end 163.083 109.417) (width 0.2) (layer "F.Cu") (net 14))
 (segment (start 167.1 105.4) (end 169.9375 105.4) (width 0.2) (layer "F.Cu") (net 14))
 (segment (start 163.083 109.417) (end 167.1 105.4) (width 0.2) (layer "F.Cu") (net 14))
 (segment (start 147.00625 111.04375) (end 148.633 109.417) (width 0.2) (layer "F.Cu") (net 14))
 (segment (start 169.9375 105.4) (end 175.58125 111.04375) (width 0.2) (layer "F.Cu") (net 14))
 (segment (start 171.3 113.6) (end 171.3754 113.6) (width 0.2) (layer "F.Cu") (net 16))
 (segment (start 171.77485 113.66725) (end 171.8421 113.6) (width 0.2) (layer "F.Cu") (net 16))
 (segment (start 174.775 113.6) (end 175.58125 112.79375) (width 0.2) (layer "F.Cu") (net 16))
 (segment (start 170.98025 113.51975) (end 171.21975 113.51975) (width 0.2) (layer "F.Cu") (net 16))
 (segment (start 143.50625 111.04375) (end 144.2625 111.8) (width 0.2) (layer "F.Cu") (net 16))
 (segment (start 144.2625 111.8) (end 169.5 111.8) (width 0.2) (layer "F.Cu") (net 16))
 (segment (start 169.5 111.8) (end 170.98025 113.28025) (width 0.2) (layer "F.Cu") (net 16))
 (segment (start 171.8421 113.6) (end 174.775 113.6) (width 0.2) (layer "F.Cu") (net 16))
 (segment (start 171.3754 113.6) (end 171.44265 113.66725) (width 0.2) (layer "F.Cu") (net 16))
 (segment (start 170.98025 113.28025) (end 170.98025 113.51975) (width 0.2) (layer "F.Cu") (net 16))
 (segment (start 171.44265 113.66725) (end 171.77485 113.66725) (width 0.2) (layer "F.Cu") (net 16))
 (segment (start 171.21975 113.51975) (end 171.3 113.6) (width 0.2) (layer "F.Cu") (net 16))
 (segment (start 171.60875 147.32) (end 171.60875 128.27) (width 0.2) (layer "F.Cu") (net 1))
 (segment (start 176.68225 112.06775) (end 172.80725 112.06775) (width 0.2) (layer "F.Cu") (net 1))
 (segment (start 172.08125 112.79375) (end 169.8 110.5125) (width 0.2) (layer "F.Cu") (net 1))
 (segment (start 169.8 110.5125) (end 169.8 109.56237) (width 0.2) (layer "F.Cu") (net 1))
 (segment (start 152.55875 128.27) (end 143.50625 119.2175) (width 0.2) (layer "F.Cu") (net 1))
 (segment (start 176.68225 123.1965) (end 176.68225 112.06775) (width 0.2) (layer "F.Cu") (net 1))
 (segment (start 168.17763 107.94) (end 167.1 107.94) (width 0.2) (layer "F.Cu") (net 1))
 (segment (start 171.60875 128.27) (end 176.68225 123.1965) (width 0.2) (layer "F.Cu") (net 1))
 (segment (start 169.8 109.56237) (end 168.17763 107.94) (width 0.2) (layer "F.Cu") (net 1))
 (segment (start 172.80725 112.06775) (end 172.08125 112.79375) (width 0.2) (layer "F.Cu") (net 1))
 (segment (start 143.50625 119.2175) (end 143.50625 112.79375) (width 0.2) (layer "F.Cu") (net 1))
 (segment (start 152.55875 147.32) (end 152.55875 128.27) (width 0.2) (layer "B.Cu") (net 1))
 (segment (start 164.54822 151.261) (end 160.60722 147.32) (width 0.2) (layer "B.Cu") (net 1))
 (segment (start 160.60722 147.32) (end 152.55875 147.32) (width 0.2) (layer "B.Cu") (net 1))
 (segment (start 165.839064 151.261) (end 164.54822 151.261) (width 0.2) (layer "B.Cu") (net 1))
 (segment (start 169.780064 147.32) (end 165.839064 151.261) (width 0.2) (layer "B.Cu") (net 1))
 (segment (start 171.60875 147.32) (end 169.780064 147.32) (width 0.2) (layer "B.Cu") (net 1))
 (segment (start 147.00625 112.79375) (end 149.7725 115.56) (width 0.2) (layer "F.Cu") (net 9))
 (segment (start 149.7725 115.56) (end 151.86 115.56) (width 0.2) (layer "F.Cu") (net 9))
 (segment (start 146.20875 130.81) (end 156.93 130.81) (width 0.2) (layer "F.Cu") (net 3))
 (segment (start 156.93 130.81) (end 167.1 120.64) (width 0.2) (layer "F.Cu") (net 3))
 (segment (start 165.25875 130.81) (end 169.452 126.61675) (width 0.2) (layer "F.Cu") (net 12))
 (segment (start 169.452 126.61675) (end 169.452 119.37437) (width 0.2) (layer "F.Cu") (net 12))
 (segment (start 169.452 119.37437) (end 168.17763 118.1) (width 0.2) (layer "F.Cu") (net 12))
 (segment (start 168.17763 118.1) (end 167.1 118.1) (width 0.2) (layer "F.Cu") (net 12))
 (segment (start 153.139064 129.671) (end 167.1 115.710064) (width 0.2) (layer "F.Cu") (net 4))
 (segment (start 146.20875 149.86) (end 146.20875 132.791314) (width 0.2) (layer "F.Cu") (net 4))
 (segment (start 144.80775 131.390314) (end 144.80775 130.229686) (width 0.2) (layer "F.Cu") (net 4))
 (segment (start 146.20875 132.791314) (end 144.80775 131.390314) (width 0.2) (layer "F.Cu") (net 4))
 (segment (start 145.628436 129.409) (end 146.789064 129.409) (width 0.2) (layer "F.Cu") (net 4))
 (segment (start 147.051064 129.671) (end 153.139064 129.671) (width 0.2) (layer "F.Cu") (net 4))
 (segment (start 146.789064 129.409) (end 147.051064 129.671) (width 0.2) (layer "F.Cu") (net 4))
 (segment (start 144.80775 130.229686) (end 145.628436 129.409) (width 0.2) (layer "F.Cu") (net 4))
 (segment (start 167.1 115.710064) (end 167.1 115.56) (width 0.2) (layer "F.Cu") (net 4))
 (segment (start 167.301126 112.395) (end 166.6875 112.395) (width 0.2) (layer "F.Cu") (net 2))
 (segment (start 166.037 114.083) (end 166.037 126.93672) (width 0.2) (layer "B.Cu") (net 2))
 (segment (start 166.71775 148.401) (end 165.25875 149.86) (width 0.2) (layer "B.Cu") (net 2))
 (segment (start 166.037 126.93672) (end 166.71775 127.61747) (width 0.2) (layer "B.Cu") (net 2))
 (segment (start 167.1 113.02) (end 166.037 114.083) (width 0.2) (layer "B.Cu") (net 2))
 (segment (start 166.71775 127.61747) (end 166.71775 148.401) (width 0.2) (layer "B.Cu") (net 2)))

